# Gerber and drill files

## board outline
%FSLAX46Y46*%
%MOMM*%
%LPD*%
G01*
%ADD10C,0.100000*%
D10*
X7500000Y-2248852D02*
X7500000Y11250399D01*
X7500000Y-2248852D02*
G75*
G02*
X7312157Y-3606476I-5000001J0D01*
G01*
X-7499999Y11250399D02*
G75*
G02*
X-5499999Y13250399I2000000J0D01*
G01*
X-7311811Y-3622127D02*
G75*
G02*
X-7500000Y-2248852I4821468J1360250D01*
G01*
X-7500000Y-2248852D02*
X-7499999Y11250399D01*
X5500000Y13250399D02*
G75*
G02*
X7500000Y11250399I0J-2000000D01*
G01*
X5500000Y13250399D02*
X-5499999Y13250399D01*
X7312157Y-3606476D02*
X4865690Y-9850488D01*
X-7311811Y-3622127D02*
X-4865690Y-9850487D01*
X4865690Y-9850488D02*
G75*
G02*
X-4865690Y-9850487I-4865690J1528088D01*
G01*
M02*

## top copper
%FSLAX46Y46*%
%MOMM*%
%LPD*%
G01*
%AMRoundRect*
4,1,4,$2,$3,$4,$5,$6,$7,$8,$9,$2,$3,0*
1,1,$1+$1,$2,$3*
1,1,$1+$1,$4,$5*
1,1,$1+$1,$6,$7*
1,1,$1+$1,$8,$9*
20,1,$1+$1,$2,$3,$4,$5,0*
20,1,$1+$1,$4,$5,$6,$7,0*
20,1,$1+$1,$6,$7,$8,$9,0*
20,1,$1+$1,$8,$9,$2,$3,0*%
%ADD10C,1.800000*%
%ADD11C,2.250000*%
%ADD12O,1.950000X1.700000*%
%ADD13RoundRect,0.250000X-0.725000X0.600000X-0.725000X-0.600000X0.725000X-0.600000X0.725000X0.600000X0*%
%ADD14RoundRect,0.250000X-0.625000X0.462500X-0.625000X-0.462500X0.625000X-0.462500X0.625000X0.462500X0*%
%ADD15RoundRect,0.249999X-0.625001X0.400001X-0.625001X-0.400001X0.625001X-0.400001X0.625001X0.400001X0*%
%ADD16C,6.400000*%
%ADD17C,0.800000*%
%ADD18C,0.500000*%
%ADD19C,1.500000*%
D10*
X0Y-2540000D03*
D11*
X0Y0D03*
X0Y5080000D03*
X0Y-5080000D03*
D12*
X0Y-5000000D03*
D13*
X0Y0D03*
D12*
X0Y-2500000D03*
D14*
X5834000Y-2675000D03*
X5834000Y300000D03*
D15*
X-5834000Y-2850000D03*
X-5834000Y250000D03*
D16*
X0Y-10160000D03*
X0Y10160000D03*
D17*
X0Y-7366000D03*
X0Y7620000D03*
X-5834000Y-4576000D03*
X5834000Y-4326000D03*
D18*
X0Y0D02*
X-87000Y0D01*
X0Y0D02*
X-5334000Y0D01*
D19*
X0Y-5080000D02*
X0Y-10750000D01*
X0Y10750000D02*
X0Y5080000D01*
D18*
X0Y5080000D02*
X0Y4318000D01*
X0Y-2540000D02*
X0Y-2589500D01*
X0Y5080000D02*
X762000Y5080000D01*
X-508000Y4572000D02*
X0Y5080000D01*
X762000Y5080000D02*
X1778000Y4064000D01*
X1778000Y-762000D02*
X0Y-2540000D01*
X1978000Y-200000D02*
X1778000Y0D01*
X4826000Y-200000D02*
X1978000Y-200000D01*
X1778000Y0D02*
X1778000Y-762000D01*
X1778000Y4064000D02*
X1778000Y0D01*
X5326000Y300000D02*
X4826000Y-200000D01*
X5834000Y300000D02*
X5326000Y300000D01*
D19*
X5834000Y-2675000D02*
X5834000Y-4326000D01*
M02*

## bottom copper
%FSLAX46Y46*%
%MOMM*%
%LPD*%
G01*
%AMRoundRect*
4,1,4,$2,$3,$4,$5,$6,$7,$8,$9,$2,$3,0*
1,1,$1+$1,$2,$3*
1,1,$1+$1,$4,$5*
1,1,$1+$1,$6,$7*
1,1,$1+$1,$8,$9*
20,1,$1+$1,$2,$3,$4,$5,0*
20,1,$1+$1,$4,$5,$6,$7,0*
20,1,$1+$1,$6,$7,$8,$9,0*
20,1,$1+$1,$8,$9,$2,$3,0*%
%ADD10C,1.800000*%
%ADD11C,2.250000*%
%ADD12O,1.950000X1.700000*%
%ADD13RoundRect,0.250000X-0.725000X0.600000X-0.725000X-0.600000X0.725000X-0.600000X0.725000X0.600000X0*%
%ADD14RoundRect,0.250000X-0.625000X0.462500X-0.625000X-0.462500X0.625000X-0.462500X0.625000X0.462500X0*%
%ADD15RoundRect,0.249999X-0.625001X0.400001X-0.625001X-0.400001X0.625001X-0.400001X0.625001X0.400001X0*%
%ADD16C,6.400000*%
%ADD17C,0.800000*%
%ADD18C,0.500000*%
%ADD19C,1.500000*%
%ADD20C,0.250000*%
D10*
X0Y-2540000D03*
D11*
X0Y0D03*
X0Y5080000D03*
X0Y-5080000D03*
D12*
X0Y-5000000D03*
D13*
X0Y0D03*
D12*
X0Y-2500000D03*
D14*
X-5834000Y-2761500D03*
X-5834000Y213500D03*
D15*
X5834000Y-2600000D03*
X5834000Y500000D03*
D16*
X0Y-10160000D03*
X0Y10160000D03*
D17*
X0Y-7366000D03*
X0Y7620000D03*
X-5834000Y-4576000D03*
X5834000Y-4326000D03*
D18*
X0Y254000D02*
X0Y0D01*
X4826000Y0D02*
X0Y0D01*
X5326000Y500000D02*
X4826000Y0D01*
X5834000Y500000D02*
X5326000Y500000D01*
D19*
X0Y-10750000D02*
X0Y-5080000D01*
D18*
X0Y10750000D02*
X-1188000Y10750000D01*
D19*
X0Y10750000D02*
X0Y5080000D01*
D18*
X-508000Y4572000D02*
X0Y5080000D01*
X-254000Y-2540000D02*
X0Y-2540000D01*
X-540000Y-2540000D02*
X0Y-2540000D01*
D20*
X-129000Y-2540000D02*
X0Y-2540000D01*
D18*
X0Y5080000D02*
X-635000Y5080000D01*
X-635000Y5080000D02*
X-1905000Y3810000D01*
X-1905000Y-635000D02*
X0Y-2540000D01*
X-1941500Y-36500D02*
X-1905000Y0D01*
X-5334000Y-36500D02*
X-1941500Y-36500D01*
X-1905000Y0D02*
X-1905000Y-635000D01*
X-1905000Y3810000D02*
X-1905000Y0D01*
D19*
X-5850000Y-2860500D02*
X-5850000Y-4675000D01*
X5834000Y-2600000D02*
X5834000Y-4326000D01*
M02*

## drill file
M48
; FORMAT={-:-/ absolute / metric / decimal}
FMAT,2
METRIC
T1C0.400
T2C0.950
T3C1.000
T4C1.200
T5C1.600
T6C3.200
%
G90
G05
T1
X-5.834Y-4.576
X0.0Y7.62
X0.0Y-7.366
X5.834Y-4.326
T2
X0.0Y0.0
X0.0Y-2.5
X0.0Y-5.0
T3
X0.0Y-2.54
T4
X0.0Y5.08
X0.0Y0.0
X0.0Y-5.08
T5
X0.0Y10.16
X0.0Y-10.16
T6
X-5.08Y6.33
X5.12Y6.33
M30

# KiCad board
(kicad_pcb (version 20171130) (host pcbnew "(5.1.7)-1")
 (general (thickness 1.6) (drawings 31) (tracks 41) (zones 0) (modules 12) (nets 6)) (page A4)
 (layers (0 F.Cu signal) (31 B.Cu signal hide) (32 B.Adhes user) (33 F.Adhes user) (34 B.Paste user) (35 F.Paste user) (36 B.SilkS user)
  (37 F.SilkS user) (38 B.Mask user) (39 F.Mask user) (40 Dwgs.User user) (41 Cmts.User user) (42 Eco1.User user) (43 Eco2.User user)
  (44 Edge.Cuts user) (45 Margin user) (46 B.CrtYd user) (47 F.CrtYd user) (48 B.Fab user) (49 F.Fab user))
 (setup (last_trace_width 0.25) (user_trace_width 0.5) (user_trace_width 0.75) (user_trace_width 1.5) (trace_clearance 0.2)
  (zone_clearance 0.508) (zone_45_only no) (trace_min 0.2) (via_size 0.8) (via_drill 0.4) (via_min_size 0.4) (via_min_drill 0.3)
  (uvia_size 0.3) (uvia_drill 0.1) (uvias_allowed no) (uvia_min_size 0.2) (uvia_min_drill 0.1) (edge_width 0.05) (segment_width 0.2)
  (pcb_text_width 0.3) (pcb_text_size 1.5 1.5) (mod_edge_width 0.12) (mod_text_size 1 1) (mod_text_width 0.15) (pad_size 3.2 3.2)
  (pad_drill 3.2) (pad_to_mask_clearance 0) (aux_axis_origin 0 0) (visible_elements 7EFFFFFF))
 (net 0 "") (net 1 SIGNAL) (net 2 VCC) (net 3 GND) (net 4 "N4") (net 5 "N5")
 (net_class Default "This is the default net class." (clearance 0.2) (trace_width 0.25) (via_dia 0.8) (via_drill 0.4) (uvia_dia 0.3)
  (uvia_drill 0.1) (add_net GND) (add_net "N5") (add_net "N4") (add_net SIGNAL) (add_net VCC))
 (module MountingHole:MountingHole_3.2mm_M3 (layer F.Cu) (at -5.08 -6.33)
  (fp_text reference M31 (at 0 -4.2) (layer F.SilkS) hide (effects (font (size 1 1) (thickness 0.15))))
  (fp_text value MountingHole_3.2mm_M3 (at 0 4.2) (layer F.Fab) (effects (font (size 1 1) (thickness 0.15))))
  (pad "" np_thru_hole circle (at 0 0) (size 3.2 3.2) (drill 3.2) (layers *.Cu *.Mask)))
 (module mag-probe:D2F (layer F.Cu) (at 0 0 270)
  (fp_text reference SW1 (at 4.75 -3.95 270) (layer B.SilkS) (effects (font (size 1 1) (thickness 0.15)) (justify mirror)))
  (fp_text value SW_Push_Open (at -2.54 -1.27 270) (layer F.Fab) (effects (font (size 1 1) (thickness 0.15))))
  (pad 4 thru_hole circle (at 2.54 0 270) (size 1.8 1.8) (drill 1) (layers *.Cu *.Mask) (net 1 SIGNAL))
  (pad 3 thru_hole circle (at 0 0 270) (size 2.25 2.25) (drill 1.2) (layers *.Cu *.Mask) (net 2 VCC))
  (pad 2 thru_hole circle (at -5.08 0 270) (size 2.25 2.25) (drill 1.2) (layers *.Cu *.Mask) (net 1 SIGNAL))
  (pad 1 thru_hole circle (at 5.08 0 270) (size 2.25 2.25) (drill 1.2) (layers *.Cu *.Mask) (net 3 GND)))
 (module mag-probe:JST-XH (layer F.Cu) (at 0 0 270)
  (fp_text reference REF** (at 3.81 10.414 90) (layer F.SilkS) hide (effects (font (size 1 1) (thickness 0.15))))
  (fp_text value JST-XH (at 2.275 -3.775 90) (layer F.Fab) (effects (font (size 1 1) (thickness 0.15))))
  (pad 3 thru_hole oval (at 5 0 270) (size 1.7 1.95) (drill 0.95) (layers *.Cu *.Mask))
  (pad 1 thru_hole roundrect (at 0 0 270) (size 1.7 1.95) (drill 0.95) (layers *.Cu *.Mask) (roundrect_rratio 0.1470588235294118))
  (pad 2 thru_hole oval (at 2.5 0 270) (size 1.7 1.95) (drill 0.95) (layers *.Cu *.Mask)))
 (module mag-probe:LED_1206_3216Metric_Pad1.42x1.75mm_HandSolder (layer F.Cu) (at 5.834 1.1875 270)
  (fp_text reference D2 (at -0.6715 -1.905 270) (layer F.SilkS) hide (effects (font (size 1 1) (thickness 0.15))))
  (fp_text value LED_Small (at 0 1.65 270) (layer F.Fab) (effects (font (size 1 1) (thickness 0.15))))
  (pad 2 smd roundrect (at 1.4875 0 270) (size 1.425 1.75) (layers F.Cu F.Paste F.Mask) (roundrect_rratio 0.1754385964912281) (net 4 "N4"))
  (pad 1 smd roundrect (at -1.4875 0 270) (size 1.425 1.75) (layers F.Cu F.Paste F.Mask) (roundrect_rratio 0.1754385964912281)
   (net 1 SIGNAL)))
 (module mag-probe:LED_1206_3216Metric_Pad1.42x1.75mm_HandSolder (layer B.Cu) (at -5.834 1.274 270)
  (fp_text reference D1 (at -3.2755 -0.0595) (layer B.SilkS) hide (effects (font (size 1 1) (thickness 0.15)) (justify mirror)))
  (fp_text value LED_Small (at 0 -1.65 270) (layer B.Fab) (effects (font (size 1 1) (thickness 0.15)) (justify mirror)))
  (pad 2 smd roundrect (at 1.4875 0 270) (size 1.425 1.75) (layers B.Cu B.Paste B.Mask) (roundrect_rratio 0.1754385964912281) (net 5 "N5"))
  (pad 1 smd roundrect (at -1.4875 0 270) (size 1.425 1.75) (layers B.Cu B.Paste B.Mask) (roundrect_rratio 0.1754385964912281)
   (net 1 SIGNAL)))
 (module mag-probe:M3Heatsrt (layer F.Cu) (at -5.08 -6.33)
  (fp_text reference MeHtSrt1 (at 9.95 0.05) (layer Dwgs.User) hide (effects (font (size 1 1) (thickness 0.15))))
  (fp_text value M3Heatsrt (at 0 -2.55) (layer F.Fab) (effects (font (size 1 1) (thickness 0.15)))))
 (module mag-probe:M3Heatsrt (layer F.Cu) (at 5.08 -6.33)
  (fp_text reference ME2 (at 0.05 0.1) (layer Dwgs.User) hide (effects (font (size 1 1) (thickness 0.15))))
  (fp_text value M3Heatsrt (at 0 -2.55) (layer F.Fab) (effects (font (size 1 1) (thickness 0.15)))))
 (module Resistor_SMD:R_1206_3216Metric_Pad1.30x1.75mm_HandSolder (layer F.Cu) (at -5.834 1.3 270)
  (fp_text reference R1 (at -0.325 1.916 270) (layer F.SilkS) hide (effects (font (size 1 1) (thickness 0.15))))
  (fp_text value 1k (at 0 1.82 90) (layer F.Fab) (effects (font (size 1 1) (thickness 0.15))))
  (pad 2 smd roundrect (at 1.55 0 270) (size 1.3 1.75) (layers F.Cu F.Paste F.Mask) (roundrect_rratio 0.1923069230769231) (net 5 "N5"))
  (pad 1 smd roundrect (at -1.55 0 270) (size 1.3 1.75) (layers F.Cu F.Paste F.Mask) (roundrect_rratio 0.1923069230769231) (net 2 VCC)))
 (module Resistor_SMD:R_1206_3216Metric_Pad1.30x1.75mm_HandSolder (layer B.Cu) (at 5.834 1.05 270)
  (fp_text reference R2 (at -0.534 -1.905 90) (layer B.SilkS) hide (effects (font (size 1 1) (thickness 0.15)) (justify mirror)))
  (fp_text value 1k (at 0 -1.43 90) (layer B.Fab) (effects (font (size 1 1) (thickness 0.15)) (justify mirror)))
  (pad 2 smd roundrect (at 1.55 0 270) (size 1.3 1.75) (layers B.Cu B.Paste B.Mask) (roundrect_rratio 0.1923069230769231) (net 4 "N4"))
  (pad 1 smd roundrect (at -1.55 0 270) (size 1.3 1.75) (layers B.Cu B.Paste B.Mask) (roundrect_rratio 0.1923069230769231) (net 2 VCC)))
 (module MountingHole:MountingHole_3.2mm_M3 (layer F.Cu) (at 5.08 -6.33)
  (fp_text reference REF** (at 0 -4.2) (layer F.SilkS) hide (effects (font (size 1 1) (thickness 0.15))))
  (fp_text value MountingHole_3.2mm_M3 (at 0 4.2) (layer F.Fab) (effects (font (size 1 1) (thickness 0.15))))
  (pad "" np_thru_hole circle (at 0.04 0) (size 3.2 3.2) (drill 3.2) (layers *.Cu *.Mask)))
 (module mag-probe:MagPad (layer F.Cu) (at 0 10.16)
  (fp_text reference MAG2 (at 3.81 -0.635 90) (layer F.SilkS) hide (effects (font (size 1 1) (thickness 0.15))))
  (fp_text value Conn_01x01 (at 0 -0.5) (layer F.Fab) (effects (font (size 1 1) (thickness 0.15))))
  (pad 1 thru_hole circle (at 0 0) (size 6.4 6.4) (drill 1.6) (layers *.Cu *.Mask) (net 3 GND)))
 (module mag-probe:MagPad (layer F.Cu) (at 0 -10.16)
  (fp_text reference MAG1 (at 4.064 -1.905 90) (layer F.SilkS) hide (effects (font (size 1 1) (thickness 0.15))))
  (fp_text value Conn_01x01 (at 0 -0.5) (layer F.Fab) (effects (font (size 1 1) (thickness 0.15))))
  (pad 1 thru_hole circle (at 0 0) (size 6.4 6.4) (drill 1.6) (layers *.Cu *.Mask) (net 1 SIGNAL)))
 (gr_line (start 7.5 2.248852) (end 7.5 -11.250399) (layer Edge.Cuts) (width 0.1))
 (gr_arc (start 2.499999 2.248852) (end 7.312157 3.606476) (angle -15.75501346) (layer Edge.Cuts) (width 0.1))
 (gr_arc (start -5.499999 -11.250399) (end -5.499999 -13.250399) (angle -90) (layer Edge.Cuts) (width 0.1))
 (gr_arc (start -2.490343 2.261877) (end -7.5 2.248852) (angle -15.90398022) (layer Edge.Cuts) (width 0.1))
 (gr_line (start -7.5 2.248852) (end -7.499999 -11.250399) (layer Edge.Cuts) (width 0.1))
 (gr_arc (start 5.5 -11.250399) (end 7.5 -11.250399) (angle -90) (layer Edge.Cuts) (width 0.1))
 (gr_line (start 5.5 -13.250399) (end -5.499999 -13.250399) (layer Edge.Cuts) (width 0.1))
 (gr_line (start 7.312157 3.606476) (end 4.86569 9.850488) (layer Edge.Cuts) (width 0.1))
 (gr_line (start -7.311811 3.622127) (end -4.86569 9.850487) (layer Edge.Cuts) (width 0.1))
 (gr_arc (start 0 8.3224) (end -4.86569 9.850487) (angle -145.1298326) (layer Edge.Cuts) (width 0.1))
 (segment (start 0 -0.254) (end 0 0) (width 0.5) (layer B.Cu) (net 2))
 (segment (start 0 0) (end -0.087 0) (width 0.5) (layer F.Cu) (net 2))
 (segment (start 4.826 0) (end 0 0) (width 0.5) (layer B.Cu) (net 2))
 (segment (start 0 0) (end -5.334 0) (width 0.5) (layer F.Cu) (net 2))
 (segment (start 5.326 -0.5) (end 4.826 0) (width 0.5) (layer B.Cu) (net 2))
 (segment (start 5.834 -0.5) (end 5.326 -0.5) (width 0.5) (layer B.Cu) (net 2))
 (segment (start 0 10.75) (end 0 5.08) (width 1.5) (layer B.Cu) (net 3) (status 30))
 (segment (start 0 5.08) (end 0 10.75) (width 1.5) (layer F.Cu) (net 3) (status 30))
 (via (at 0 7.366) (size 0.8) (drill 0.4) (layers F.Cu B.Cu) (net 3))
 (via (at 0 -7.62) (size 0.8) (drill 0.4) (layers F.Cu B.Cu) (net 1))
 (segment (start 0 -10.75) (end -1.188 -10.75) (width 0.5) (layer B.Cu) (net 1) (status 30))
 (segment (start 0 -10.75) (end 0 -5.08) (width 1.5) (layer B.Cu) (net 1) (status 30))
 (segment (start -0.508 -4.572) (end 0 -5.08) (width 0.5) (layer B.Cu) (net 1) (status 30))
 (segment (start 0 -10.75) (end 0 -5.08) (width 1.5) (layer F.Cu) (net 1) (status 30))
 (segment (start -0.254 2.54) (end 0 2.54) (width 0.5) (layer B.Cu) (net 1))
 (segment (start 0 -5.08) (end 0 -4.318) (width 0.5) (layer F.Cu) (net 1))
 (segment (start 0 2.54) (end 0 2.5895) (width 0.5) (layer F.Cu) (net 1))
 (segment (start -0.54 2.54) (end 0 2.54) (width 0.5) (layer B.Cu) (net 1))
 (segment (start -0.129 2.54) (end 0 2.54) (width 0.25) (layer B.Cu) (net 1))
 (segment (start 0 -5.08) (end 0.762 -5.08) (width 0.5) (layer F.Cu) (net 1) (status 30))
 (segment (start -0.508 -4.572) (end 0 -5.08) (width 0.5) (layer F.Cu) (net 1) (status 30))
 (segment (start 0 -5.08) (end -0.635 -5.08) (width 0.5) (layer B.Cu) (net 1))
 (segment (start -0.635 -5.08) (end -1.905 -3.81) (width 0.5) (layer B.Cu) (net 1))
 (segment (start -1.905 0.635) (end 0 2.54) (width 0.5) (layer B.Cu) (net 1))
 (segment (start 0.762 -5.08) (end 1.778 -4.064) (width 0.5) (layer F.Cu) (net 1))
 (segment (start 1.778 0.762) (end 0 2.54) (width 0.5) (layer F.Cu) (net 1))
 (segment (start 1.978 0.2) (end 1.778 0) (width 0.5) (layer F.Cu) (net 1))
 (segment (start 4.826 0.2) (end 1.978 0.2) (width 0.5) (layer F.Cu) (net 1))
 (segment (start 1.778 0) (end 1.778 0.762) (width 0.5) (layer F.Cu) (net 1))
 (segment (start 1.778 -4.064) (end 1.778 0) (width 0.5) (layer F.Cu) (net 1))
 (segment (start -1.9415 0.0365) (end -1.905 0) (width 0.5) (layer B.Cu) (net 1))
 (segment (start -5.334 0.0365) (end -1.9415 0.0365) (width 0.5) (layer B.Cu) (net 1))
 (segment (start -1.905 0) (end -1.905 0.635) (width 0.5) (layer B.Cu) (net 1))
 (segment (start -1.905 -3.81) (end -1.905 0) (width 0.5) (layer B.Cu) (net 1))
 (segment (start 5.326 -0.3) (end 4.826 0.2) (width 0.5) (layer F.Cu) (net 1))
 (segment (start 5.834 -0.3) (end 5.326 -0.3) (width 0.5) (layer F.Cu) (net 1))
 (via (at -5.834 4.576) (size 0.8) (drill 0.4) (layers F.Cu B.Cu) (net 5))
 (segment (start -5.85 2.8605) (end -5.85 4.675) (width 1.5) (layer B.Cu) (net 5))
 (via (at 5.834 4.326) (size 0.8) (drill 0.4) (layers F.Cu B.Cu) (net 4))
 (segment (start 5.834 2.6) (end 5.834 4.326) (width 1.5) (layer B.Cu) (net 4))
 (segment (start 5.834 2.675) (end 5.834 4.326) (width 1.5) (layer F.Cu) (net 4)))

